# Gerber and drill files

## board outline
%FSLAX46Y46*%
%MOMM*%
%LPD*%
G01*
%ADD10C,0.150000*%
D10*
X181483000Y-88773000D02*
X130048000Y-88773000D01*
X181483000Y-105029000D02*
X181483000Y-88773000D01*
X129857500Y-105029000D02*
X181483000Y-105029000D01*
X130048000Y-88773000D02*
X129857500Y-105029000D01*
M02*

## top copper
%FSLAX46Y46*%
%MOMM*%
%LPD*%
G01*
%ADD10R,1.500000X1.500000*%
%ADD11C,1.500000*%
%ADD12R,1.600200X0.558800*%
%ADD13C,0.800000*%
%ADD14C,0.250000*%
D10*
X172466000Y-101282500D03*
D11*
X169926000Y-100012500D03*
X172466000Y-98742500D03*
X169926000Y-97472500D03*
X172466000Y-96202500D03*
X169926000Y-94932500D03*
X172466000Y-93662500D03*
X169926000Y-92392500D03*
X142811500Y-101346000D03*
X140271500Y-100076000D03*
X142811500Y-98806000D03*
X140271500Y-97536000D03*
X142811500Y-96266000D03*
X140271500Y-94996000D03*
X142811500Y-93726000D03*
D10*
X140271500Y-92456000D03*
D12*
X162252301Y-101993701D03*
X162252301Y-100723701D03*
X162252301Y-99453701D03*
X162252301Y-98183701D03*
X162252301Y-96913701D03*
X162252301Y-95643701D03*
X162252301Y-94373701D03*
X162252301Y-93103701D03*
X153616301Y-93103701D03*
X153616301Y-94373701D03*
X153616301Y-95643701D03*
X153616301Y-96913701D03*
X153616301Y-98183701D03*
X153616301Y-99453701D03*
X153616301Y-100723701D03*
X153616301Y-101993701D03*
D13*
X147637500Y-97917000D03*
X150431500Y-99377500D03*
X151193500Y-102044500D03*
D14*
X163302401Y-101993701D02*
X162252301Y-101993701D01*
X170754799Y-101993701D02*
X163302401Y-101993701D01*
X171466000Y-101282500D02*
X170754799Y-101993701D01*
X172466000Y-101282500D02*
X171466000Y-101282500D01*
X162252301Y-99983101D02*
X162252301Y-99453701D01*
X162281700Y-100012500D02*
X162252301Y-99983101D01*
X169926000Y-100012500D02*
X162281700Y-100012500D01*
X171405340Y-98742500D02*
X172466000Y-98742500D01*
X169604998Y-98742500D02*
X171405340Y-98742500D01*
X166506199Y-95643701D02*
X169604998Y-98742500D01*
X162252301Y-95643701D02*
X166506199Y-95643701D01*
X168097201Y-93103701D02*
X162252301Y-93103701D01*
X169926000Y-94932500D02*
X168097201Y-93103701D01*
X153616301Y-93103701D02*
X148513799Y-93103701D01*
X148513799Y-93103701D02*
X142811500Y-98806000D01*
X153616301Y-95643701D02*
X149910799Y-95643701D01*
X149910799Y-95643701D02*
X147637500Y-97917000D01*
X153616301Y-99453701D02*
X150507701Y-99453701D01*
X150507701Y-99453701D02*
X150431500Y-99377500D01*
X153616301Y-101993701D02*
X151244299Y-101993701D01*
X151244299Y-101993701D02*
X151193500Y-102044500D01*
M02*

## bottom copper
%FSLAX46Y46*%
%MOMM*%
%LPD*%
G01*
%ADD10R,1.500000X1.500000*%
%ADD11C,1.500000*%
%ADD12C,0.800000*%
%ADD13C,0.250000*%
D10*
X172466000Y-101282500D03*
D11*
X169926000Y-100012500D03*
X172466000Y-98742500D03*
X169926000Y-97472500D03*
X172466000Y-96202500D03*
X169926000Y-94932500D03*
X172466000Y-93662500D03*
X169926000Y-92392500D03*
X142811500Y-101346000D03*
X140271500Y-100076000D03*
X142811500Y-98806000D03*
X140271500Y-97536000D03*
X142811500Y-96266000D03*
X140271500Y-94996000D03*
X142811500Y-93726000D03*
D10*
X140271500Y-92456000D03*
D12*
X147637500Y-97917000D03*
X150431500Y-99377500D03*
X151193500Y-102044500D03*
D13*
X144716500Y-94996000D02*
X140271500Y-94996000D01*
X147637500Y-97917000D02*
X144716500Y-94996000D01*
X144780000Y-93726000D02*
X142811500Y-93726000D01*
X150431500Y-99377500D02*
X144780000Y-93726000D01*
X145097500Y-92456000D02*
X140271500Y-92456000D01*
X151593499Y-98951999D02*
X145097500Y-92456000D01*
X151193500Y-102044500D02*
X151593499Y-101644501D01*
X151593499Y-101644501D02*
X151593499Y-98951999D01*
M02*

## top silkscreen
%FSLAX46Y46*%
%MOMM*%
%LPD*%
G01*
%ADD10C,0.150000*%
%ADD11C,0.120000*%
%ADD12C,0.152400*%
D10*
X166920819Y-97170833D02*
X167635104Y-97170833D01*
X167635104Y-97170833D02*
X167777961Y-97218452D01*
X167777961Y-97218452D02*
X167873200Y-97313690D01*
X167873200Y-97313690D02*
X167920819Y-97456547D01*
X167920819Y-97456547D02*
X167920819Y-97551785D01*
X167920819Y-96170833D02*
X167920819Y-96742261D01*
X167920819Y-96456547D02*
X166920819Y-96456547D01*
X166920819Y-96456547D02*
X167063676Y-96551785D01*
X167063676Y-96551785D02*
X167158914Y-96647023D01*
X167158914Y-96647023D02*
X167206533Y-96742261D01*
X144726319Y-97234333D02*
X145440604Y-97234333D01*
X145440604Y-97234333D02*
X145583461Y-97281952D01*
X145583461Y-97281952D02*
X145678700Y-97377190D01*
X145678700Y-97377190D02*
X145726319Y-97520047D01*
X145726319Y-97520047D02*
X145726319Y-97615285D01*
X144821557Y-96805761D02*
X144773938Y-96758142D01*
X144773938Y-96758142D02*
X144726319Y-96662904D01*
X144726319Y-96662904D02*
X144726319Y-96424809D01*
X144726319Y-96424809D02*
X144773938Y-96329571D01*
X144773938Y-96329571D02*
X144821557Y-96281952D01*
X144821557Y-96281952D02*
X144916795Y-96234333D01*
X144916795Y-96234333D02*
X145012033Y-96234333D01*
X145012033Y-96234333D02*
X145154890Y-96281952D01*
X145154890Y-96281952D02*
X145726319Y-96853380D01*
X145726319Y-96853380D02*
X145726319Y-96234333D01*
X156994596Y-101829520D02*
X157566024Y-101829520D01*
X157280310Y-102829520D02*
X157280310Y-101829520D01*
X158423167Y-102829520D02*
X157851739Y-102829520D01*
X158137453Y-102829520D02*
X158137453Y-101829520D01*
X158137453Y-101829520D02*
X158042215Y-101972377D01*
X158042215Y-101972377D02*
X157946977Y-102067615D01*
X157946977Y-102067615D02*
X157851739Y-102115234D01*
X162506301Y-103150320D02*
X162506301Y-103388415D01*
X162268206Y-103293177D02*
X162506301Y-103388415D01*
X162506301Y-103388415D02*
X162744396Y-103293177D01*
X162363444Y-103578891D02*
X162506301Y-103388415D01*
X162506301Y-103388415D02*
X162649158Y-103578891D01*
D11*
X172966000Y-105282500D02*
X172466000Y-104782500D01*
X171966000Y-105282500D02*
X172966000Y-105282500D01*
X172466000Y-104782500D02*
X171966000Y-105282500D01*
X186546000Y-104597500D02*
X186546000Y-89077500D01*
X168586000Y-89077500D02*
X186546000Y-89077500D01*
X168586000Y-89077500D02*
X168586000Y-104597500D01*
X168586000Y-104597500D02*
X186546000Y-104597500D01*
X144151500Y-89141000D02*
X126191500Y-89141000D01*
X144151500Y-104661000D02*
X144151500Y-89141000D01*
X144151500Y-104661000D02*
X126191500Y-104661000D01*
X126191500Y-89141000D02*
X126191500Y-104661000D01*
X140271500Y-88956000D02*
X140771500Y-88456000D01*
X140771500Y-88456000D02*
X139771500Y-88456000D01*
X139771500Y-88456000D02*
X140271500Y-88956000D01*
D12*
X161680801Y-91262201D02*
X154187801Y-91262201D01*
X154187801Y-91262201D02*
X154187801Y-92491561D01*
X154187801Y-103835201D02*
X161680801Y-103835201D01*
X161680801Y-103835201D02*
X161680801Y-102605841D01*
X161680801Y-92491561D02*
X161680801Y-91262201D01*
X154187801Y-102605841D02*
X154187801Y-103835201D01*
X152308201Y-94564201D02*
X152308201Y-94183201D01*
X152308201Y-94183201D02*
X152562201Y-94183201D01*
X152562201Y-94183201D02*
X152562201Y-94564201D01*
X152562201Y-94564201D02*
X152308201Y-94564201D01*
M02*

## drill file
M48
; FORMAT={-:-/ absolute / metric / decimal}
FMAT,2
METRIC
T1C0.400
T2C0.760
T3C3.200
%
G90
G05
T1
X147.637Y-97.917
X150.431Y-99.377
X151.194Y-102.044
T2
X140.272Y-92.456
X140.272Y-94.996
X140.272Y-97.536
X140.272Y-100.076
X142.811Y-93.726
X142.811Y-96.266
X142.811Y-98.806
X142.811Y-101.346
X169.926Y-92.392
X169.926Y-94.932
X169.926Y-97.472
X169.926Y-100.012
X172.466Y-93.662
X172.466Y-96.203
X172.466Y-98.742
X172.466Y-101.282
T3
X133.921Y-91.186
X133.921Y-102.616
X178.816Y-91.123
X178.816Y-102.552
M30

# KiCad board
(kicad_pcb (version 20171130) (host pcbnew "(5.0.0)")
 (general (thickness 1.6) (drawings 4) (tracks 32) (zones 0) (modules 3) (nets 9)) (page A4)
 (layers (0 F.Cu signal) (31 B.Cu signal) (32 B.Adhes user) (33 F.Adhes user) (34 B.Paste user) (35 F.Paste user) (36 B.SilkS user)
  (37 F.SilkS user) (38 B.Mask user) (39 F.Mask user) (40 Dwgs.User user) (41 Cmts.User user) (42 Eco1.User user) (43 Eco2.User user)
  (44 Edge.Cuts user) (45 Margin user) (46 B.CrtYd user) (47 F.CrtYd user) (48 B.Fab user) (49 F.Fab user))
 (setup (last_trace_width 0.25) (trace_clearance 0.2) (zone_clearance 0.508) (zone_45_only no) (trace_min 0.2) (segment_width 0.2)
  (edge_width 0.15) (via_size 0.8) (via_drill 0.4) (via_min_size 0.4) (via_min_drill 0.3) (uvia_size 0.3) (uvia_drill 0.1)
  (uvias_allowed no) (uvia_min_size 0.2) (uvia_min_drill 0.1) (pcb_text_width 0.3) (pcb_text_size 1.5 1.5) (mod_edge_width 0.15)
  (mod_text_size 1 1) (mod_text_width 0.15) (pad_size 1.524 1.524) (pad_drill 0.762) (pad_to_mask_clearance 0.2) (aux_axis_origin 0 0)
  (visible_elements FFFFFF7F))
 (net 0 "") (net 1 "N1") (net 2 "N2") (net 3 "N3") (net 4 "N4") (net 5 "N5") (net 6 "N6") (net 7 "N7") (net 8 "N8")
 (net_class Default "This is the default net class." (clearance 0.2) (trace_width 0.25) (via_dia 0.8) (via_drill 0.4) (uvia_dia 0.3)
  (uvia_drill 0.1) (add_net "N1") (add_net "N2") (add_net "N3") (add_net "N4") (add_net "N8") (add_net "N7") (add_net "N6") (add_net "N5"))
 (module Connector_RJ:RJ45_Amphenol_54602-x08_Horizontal (layer F.Cu) (at 172.466 101.2825 90)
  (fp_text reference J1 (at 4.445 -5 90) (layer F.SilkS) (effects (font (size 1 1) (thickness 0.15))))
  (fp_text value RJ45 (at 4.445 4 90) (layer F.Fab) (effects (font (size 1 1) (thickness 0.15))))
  (fp_line (start -4 0.5) (end -3.5 0) (layer F.SilkS) (width 0.12))
  (fp_line (start -4 -0.5) (end -4 0.5) (layer F.SilkS) (width 0.12))
  (fp_line (start -3.5 0) (end -4 -0.5) (layer F.SilkS) (width 0.12))
  (fp_line (start -3.315 14.08) (end 12.205 14.08) (layer F.SilkS) (width 0.12))
  (fp_line (start 12.205 -3.88) (end 12.205 14.08) (layer F.SilkS) (width 0.12))
  (fp_line (start 12.205 -3.88) (end -3.315 -3.88) (layer F.SilkS) (width 0.12))
  (fp_line (start -3.315 -3.88) (end -3.315 14.08) (layer F.SilkS) (width 0.12))
  (pad "" np_thru_hole circle (at 10.16 6.35 90) (size 3.2 3.2) (drill 3.2) (layers *.Cu *.Mask))
  (pad "" np_thru_hole circle (at -1.27 6.35 90) (size 3.2 3.2) (drill 3.2) (layers *.Cu *.Mask))
  (pad 1 thru_hole rect (at 0 0 90) (size 1.5 1.5) (drill 0.76) (layers *.Cu *.Mask) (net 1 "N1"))
  (pad 2 thru_hole circle (at 1.27 -2.54 90) (size 1.5 1.5) (drill 0.76) (layers *.Cu *.Mask) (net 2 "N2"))
  (pad 3 thru_hole circle (at 2.54 0 90) (size 1.5 1.5) (drill 0.76) (layers *.Cu *.Mask) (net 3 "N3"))
  (pad 4 thru_hole circle (at 3.81 -2.54 90) (size 1.5 1.5) (drill 0.76) (layers *.Cu *.Mask))
  (pad 5 thru_hole circle (at 5.08 0 90) (size 1.5 1.5) (drill 0.76) (layers *.Cu *.Mask))
  (pad 6 thru_hole circle (at 6.35 -2.54 90) (size 1.5 1.5) (drill 0.76) (layers *.Cu *.Mask) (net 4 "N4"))
  (pad 7 thru_hole circle (at 7.62 0 90) (size 1.5 1.5) (drill 0.76) (layers *.Cu *.Mask))
  (pad 8 thru_hole circle (at 8.89 -2.54 90) (size 1.5 1.5) (drill 0.76) (layers *.Cu *.Mask)))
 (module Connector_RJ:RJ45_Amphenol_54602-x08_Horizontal (layer F.Cu) (at 140.2715 92.456 270)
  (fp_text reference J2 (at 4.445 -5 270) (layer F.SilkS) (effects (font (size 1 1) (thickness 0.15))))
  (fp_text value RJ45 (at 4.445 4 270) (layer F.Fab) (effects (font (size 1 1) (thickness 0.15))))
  (fp_line (start -3.315 -3.88) (end -3.315 14.08) (layer F.SilkS) (width 0.12))
  (fp_line (start 12.205 -3.88) (end -3.315 -3.88) (layer F.SilkS) (width 0.12))
  (fp_line (start 12.205 -3.88) (end 12.205 14.08) (layer F.SilkS) (width 0.12))
  (fp_line (start -3.315 14.08) (end 12.205 14.08) (layer F.SilkS) (width 0.12))
  (fp_line (start -3.5 0) (end -4 -0.5) (layer F.SilkS) (width 0.12))
  (fp_line (start -4 -0.5) (end -4 0.5) (layer F.SilkS) (width 0.12))
  (fp_line (start -4 0.5) (end -3.5 0) (layer F.SilkS) (width 0.12))
  (pad 8 thru_hole circle (at 8.89 -2.54 270) (size 1.5 1.5) (drill 0.76) (layers *.Cu *.Mask))
  (pad 7 thru_hole circle (at 7.62 0 270) (size 1.5 1.5) (drill 0.76) (layers *.Cu *.Mask))
  (pad 6 thru_hole circle (at 6.35 -2.54 270) (size 1.5 1.5) (drill 0.76) (layers *.Cu *.Mask) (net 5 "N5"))
  (pad 5 thru_hole circle (at 5.08 0 270) (size 1.5 1.5) (drill 0.76) (layers *.Cu *.Mask))
  (pad 4 thru_hole circle (at 3.81 -2.54 270) (size 1.5 1.5) (drill 0.76) (layers *.Cu *.Mask))
  (pad 3 thru_hole circle (at 2.54 0 270) (size 1.5 1.5) (drill 0.76) (layers *.Cu *.Mask) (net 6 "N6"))
  (pad 2 thru_hole circle (at 1.27 -2.54 270) (size 1.5 1.5) (drill 0.76) (layers *.Cu *.Mask) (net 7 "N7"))
  (pad 1 thru_hole rect (at 0 0 270) (size 1.5 1.5) (drill 0.76) (layers *.Cu *.Mask) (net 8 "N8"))
  (pad "" np_thru_hole circle (at -1.27 6.35 270) (size 3.2 3.2) (drill 3.2) (layers *.Cu *.Mask))
  (pad "" np_thru_hole circle (at 10.16 6.35 270) (size 3.2 3.2) (drill 3.2) (layers *.Cu *.Mask)))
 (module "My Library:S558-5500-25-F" (layer F.Cu) (at 157.934301 97.548701 180)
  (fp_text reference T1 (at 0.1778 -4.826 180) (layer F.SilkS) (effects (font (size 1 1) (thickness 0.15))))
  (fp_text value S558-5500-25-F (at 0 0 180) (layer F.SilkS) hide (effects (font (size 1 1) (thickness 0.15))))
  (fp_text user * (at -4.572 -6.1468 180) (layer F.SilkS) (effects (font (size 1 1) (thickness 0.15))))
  (fp_line (start -3.7465 6.2865) (end 3.7465 6.2865) (layer F.SilkS) (width 0.1524))
  (fp_line (start 3.7465 6.2865) (end 3.7465 5.05714) (layer F.SilkS) (width 0.1524))
  (fp_line (start 3.7465 -6.2865) (end -3.7465 -6.2865) (layer F.SilkS) (width 0.1524))
  (fp_line (start -3.7465 -6.2865) (end -3.7465 -5.05714) (layer F.SilkS) (width 0.1524))
  (fp_line (start -3.7465 5.05714) (end -3.7465 6.2865) (layer F.SilkS) (width 0.1524))
  (fp_line (start 3.7465 -5.05714) (end 3.7465 -6.2865) (layer F.SilkS) (width 0.1524))
  (fp_line (start 5.6261 2.9845) (end 5.6261 3.3655) (layer F.SilkS) (width 0.1524))
  (fp_line (start 5.6261 3.3655) (end 5.3721 3.3655) (layer F.SilkS) (width 0.1524))
  (fp_line (start 5.3721 3.3655) (end 5.3721 2.9845) (layer F.SilkS) (width 0.1524))
  (fp_line (start 5.3721 2.9845) (end 5.6261 2.9845) (layer F.SilkS) (width 0.1524))
  (pad 1 smd rect (at -4.318 -4.445 180) (size 1.6002 0.5588) (layers F.Cu F.Paste F.Mask) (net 1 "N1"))
  (pad 2 smd rect (at -4.318 -3.175 180) (size 1.6002 0.5588) (layers F.Cu F.Paste F.Mask))
  (pad 3 smd rect (at -4.318 -1.905 180) (size 1.6002 0.5588) (layers F.Cu F.Paste F.Mask) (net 2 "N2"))
  (pad 4 smd rect (at -4.318 -0.635 180) (size 1.6002 0.5588) (layers F.Cu F.Paste F.Mask))
  (pad 5 smd rect (at -4.318 0.635 180) (size 1.6002 0.5588) (layers F.Cu F.Paste F.Mask))
  (pad 6 smd rect (at -4.318 1.905 180) (size 1.6002 0.5588) (layers F.Cu F.Paste F.Mask) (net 3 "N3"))
  (pad 7 smd rect (at -4.318 3.175 180) (size 1.6002 0.5588) (layers F.Cu F.Paste F.Mask))
  (pad 8 smd rect (at -4.318 4.445 180) (size 1.6002 0.5588) (layers F.Cu F.Paste F.Mask) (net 4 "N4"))
  (pad 9 smd rect (at 4.318 4.445 180) (size 1.6002 0.5588) (layers F.Cu F.Paste F.Mask) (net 5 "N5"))
  (pad 10 smd rect (at 4.318 3.175 180) (size 1.6002 0.5588) (layers F.Cu F.Paste F.Mask))
  (pad 11 smd rect (at 4.318 1.905 180) (size 1.6002 0.5588) (layers F.Cu F.Paste F.Mask) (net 6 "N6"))
  (pad 12 smd rect (at 4.318 0.635 180) (size 1.6002 0.5588) (layers F.Cu F.Paste F.Mask))
  (pad 13 smd rect (at 4.318 -0.635 180) (size 1.6002 0.5588) (layers F.Cu F.Paste F.Mask))
  (pad 14 smd rect (at 4.318 -1.905 180) (size 1.6002 0.5588) (layers F.Cu F.Paste F.Mask) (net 7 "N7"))
  (pad 15 smd rect (at 4.318 -3.175 180) (size 1.6002 0.5588) (layers F.Cu F.Paste F.Mask))
  (pad 16 smd rect (at 4.318 -4.445 180) (size 1.6002 0.5588) (layers F.Cu F.Paste F.Mask) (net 8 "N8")))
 (gr_line (start 181.483 88.773) (end 130.048 88.773) (layer Edge.Cuts) (width 0.15))
 (gr_line (start 181.483 105.029) (end 181.483 88.773) (layer Edge.Cuts) (width 0.15))
 (gr_line (start 129.8575 105.029) (end 181.483 105.029) (layer Edge.Cuts) (width 0.15))
 (gr_line (start 130.048 88.773) (end 129.8575 105.029) (layer Edge.Cuts) (width 0.15))
 (segment (start 163.302401 101.993701) (end 162.252301 101.993701) (width 0.25) (layer F.Cu) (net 1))
 (segment (start 170.754799 101.993701) (end 163.302401 101.993701) (width 0.25) (layer F.Cu) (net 1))
 (segment (start 171.466 101.2825) (end 170.754799 101.993701) (width 0.25) (layer F.Cu) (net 1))
 (segment (start 172.466 101.2825) (end 171.466 101.2825) (width 0.25) (layer F.Cu) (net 1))
 (segment (start 162.252301 99.983101) (end 162.252301 99.453701) (width 0.25) (layer F.Cu) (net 2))
 (segment (start 162.2817 100.0125) (end 162.252301 99.983101) (width 0.25) (layer F.Cu) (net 2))
 (segment (start 169.926 100.0125) (end 162.2817 100.0125) (width 0.25) (layer F.Cu) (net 2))
 (segment (start 171.40534 98.7425) (end 172.466 98.7425) (width 0.25) (layer F.Cu) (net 3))
 (segment (start 169.604998 98.7425) (end 171.40534 98.7425) (width 0.25) (layer F.Cu) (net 3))
 (segment (start 166.506199 95.643701) (end 169.604998 98.7425) (width 0.25) (layer F.Cu) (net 3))
 (segment (start 162.252301 95.643701) (end 166.506199 95.643701) (width 0.25) (layer F.Cu) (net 3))
 (segment (start 168.097201 93.103701) (end 162.252301 93.103701) (width 0.25) (layer F.Cu) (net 4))
 (segment (start 169.926 94.9325) (end 168.097201 93.103701) (width 0.25) (layer F.Cu) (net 4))
 (segment (start 153.616301 93.103701) (end 148.513799 93.103701) (width 0.25) (layer F.Cu) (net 5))
 (segment (start 148.513799 93.103701) (end 142.8115 98.806) (width 0.25) (layer F.Cu) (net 5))
 (via (at 147.6375 97.917) (size 0.8) (drill 0.4) (layers F.Cu B.Cu) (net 6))
 (segment (start 153.616301 95.643701) (end 149.910799 95.643701) (width 0.25) (layer F.Cu) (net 6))
 (segment (start 149.910799 95.643701) (end 147.6375 97.917) (width 0.25) (layer F.Cu) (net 6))
 (segment (start 144.7165 94.996) (end 140.2715 94.996) (width 0.25) (layer B.Cu) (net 6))
 (segment (start 147.6375 97.917) (end 144.7165 94.996) (width 0.25) (layer B.Cu) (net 6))
 (via (at 150.4315 99.3775) (size 0.8) (drill 0.4) (layers F.Cu B.Cu) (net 7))
 (segment (start 153.616301 99.453701) (end 150.507701 99.453701) (width 0.25) (layer F.Cu) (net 7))
 (segment (start 150.507701 99.453701) (end 150.4315 99.3775) (width 0.25) (layer F.Cu) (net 7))
 (segment (start 144.78 93.726) (end 142.8115 93.726) (width 0.25) (layer B.Cu) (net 7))
 (segment (start 150.4315 99.3775) (end 144.78 93.726) (width 0.25) (layer B.Cu) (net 7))
 (via (at 151.1935 102.0445) (size 0.8) (drill 0.4) (layers F.Cu B.Cu) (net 8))
 (segment (start 153.616301 101.993701) (end 151.244299 101.993701) (width 0.25) (layer F.Cu) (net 8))
 (segment (start 151.244299 101.993701) (end 151.1935 102.0445) (width 0.25) (layer F.Cu) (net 8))
 (segment (start 145.0975 92.456) (end 140.2715 92.456) (width 0.25) (layer B.Cu) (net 8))
 (segment (start 151.593499 98.951999) (end 145.0975 92.456) (width 0.25) (layer B.Cu) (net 8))
 (segment (start 151.1935 102.0445) (end 151.593499 101.644501) (width 0.25) (layer B.Cu) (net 8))
 (segment (start 151.593499 101.644501) (end 151.593499 98.951999) (width 0.25) (layer B.Cu) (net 8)))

